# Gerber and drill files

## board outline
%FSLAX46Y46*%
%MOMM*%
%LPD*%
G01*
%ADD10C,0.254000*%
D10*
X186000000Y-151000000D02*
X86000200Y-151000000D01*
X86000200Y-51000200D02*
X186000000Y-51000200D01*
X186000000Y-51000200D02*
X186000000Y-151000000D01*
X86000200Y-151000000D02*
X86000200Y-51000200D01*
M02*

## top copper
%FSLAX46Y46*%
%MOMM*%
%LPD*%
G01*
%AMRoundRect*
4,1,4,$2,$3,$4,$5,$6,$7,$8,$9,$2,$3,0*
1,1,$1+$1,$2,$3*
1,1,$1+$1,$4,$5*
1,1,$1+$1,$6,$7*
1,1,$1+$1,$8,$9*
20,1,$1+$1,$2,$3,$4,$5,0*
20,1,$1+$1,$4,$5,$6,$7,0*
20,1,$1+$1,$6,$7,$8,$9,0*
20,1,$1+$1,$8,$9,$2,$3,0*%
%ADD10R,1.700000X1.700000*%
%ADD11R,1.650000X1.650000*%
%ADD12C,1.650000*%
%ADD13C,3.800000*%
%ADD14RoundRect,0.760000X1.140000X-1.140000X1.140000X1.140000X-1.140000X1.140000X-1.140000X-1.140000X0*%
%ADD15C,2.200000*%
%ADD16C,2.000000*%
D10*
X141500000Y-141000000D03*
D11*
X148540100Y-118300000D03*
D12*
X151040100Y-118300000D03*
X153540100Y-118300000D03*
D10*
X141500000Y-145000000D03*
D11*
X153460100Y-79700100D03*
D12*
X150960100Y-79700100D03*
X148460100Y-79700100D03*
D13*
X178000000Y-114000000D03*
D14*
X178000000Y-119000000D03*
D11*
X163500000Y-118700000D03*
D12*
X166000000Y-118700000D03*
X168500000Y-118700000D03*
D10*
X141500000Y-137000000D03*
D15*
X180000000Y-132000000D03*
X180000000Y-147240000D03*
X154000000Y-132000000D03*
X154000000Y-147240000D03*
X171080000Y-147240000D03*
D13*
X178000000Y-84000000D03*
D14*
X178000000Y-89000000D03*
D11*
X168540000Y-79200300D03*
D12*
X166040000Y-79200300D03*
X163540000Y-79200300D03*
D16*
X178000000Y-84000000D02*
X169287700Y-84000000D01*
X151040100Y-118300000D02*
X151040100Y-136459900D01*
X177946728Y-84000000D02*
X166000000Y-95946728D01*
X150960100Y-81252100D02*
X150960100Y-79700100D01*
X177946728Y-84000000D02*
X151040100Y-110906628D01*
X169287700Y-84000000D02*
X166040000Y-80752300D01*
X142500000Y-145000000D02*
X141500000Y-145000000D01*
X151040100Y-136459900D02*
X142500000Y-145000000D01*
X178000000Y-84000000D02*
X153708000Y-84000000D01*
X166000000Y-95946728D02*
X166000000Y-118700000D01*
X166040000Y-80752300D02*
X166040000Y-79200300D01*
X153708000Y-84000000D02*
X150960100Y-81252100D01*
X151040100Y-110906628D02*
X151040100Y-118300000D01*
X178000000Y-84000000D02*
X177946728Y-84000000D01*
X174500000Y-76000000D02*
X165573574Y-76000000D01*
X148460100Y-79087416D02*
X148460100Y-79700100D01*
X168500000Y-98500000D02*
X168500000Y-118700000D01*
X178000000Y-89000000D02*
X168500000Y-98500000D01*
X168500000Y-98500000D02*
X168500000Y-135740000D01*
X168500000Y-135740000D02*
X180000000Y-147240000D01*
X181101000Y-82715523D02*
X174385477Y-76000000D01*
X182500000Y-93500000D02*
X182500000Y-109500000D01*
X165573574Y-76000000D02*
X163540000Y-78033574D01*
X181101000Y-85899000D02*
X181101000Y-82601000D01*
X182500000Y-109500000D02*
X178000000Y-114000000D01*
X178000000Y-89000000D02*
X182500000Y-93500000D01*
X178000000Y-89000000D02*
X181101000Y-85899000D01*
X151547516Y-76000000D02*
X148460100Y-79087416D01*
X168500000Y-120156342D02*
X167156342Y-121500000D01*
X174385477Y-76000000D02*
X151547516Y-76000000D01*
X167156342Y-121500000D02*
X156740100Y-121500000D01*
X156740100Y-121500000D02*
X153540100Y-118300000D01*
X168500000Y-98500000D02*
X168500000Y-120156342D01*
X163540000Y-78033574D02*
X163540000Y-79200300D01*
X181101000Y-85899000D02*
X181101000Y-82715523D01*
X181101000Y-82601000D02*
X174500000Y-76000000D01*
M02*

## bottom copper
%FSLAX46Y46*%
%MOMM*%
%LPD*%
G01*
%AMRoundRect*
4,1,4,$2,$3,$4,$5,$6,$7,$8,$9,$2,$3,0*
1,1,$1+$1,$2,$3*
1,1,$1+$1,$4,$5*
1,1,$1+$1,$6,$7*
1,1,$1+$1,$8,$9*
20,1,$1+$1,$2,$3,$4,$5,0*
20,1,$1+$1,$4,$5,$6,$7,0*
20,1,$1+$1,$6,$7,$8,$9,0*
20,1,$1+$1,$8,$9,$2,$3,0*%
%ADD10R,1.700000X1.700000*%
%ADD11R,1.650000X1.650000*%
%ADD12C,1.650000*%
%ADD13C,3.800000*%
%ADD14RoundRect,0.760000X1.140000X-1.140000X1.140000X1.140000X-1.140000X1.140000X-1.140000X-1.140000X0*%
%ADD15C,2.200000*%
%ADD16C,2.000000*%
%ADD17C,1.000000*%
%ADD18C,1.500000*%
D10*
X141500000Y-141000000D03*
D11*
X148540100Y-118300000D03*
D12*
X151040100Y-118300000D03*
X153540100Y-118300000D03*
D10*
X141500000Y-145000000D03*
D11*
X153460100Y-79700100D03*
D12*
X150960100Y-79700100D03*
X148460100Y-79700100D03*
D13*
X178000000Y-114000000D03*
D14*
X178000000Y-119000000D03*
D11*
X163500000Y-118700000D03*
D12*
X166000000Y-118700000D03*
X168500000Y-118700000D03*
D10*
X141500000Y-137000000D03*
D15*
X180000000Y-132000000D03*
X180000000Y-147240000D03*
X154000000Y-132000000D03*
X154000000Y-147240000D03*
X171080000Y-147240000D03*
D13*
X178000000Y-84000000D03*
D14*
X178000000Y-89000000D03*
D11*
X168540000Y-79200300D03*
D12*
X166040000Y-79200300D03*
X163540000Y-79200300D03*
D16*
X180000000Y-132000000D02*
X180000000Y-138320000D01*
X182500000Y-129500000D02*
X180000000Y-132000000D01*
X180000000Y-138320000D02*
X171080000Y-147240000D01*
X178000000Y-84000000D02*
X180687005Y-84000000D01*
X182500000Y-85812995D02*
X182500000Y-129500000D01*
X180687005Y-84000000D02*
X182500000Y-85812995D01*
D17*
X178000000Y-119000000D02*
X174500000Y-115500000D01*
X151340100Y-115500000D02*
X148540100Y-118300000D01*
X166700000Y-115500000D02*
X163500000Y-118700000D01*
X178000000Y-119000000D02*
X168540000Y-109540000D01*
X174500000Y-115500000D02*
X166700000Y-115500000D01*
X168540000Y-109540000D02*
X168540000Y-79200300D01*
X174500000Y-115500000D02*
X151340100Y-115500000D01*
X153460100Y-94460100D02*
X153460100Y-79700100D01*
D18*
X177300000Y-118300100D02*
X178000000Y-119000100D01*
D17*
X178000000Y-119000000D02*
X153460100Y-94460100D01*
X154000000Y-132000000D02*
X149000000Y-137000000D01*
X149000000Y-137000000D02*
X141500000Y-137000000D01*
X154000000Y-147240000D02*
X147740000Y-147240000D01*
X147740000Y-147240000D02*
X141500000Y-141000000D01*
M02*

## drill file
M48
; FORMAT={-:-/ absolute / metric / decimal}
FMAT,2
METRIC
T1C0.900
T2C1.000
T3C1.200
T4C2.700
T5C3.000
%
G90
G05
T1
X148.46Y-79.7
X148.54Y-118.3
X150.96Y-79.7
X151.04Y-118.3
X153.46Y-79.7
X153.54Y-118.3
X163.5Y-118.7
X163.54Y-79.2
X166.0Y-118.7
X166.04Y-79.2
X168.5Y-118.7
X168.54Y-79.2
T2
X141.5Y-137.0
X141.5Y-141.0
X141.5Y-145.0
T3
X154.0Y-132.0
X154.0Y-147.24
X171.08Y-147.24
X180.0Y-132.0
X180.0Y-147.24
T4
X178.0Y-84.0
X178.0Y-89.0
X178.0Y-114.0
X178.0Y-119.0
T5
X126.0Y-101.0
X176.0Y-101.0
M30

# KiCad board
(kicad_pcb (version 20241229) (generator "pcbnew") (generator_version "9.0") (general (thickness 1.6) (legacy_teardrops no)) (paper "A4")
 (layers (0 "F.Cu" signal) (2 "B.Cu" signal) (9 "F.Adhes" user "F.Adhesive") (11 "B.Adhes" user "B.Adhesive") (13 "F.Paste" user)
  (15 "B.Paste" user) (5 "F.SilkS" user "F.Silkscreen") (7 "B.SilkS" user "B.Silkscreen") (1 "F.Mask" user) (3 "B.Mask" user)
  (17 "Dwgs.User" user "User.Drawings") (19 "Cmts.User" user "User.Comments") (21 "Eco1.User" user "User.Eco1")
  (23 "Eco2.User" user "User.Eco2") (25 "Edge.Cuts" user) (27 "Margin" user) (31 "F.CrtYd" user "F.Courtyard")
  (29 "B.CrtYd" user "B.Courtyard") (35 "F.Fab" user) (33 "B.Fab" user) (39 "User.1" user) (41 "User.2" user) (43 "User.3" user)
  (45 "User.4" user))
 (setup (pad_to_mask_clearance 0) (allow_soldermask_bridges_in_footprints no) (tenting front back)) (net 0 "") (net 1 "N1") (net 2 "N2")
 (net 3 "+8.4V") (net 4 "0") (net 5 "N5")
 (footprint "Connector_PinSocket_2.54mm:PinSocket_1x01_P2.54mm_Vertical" (layer "F.Cu") (at 141.5 141 90)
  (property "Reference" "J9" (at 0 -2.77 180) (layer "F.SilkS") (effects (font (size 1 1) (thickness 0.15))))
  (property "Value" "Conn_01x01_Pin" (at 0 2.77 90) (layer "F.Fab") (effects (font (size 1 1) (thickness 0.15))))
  (pad "1" thru_hole rect (at 0 0 90) (size 1.7 1.7) (drill 1) (layers "*.Cu" "*.Mask") (remove_unused_layers no) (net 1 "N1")))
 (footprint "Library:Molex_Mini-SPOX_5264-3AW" (layer "F.Cu") (at 148.5401 118.3)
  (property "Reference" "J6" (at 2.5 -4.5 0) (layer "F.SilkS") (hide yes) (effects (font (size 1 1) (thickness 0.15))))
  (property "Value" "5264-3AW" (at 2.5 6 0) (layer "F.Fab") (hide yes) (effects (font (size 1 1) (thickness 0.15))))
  (pad "1" thru_hole rect (at 0 0) (size 1.65 1.65) (drill 0.9) (layers "*.Cu" "*.Mask") (remove_unused_layers no) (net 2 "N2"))
  (pad "2" thru_hole circle (at 2.5 0) (size 1.65 1.65) (drill 0.9) (layers "*.Cu" "*.Mask") (remove_unused_layers no) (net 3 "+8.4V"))
  (pad "3" thru_hole circle (at 5 0) (size 1.65 1.65) (drill 0.9) (layers "*.Cu" "*.Mask") (remove_unused_layers no) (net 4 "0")))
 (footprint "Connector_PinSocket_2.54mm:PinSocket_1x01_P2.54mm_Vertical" (layer "F.Cu") (at 141.5 145 90)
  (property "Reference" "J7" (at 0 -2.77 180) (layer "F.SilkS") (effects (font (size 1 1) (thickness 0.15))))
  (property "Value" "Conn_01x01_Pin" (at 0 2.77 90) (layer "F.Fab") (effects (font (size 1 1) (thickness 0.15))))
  (pad "1" thru_hole rect (at 0 0 90) (size 1.7 1.7) (drill 1) (layers "*.Cu" "*.Mask") (remove_unused_layers no) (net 3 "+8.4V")))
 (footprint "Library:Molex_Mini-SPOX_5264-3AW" (layer "F.Cu") (at 153.4601 79.7001 180)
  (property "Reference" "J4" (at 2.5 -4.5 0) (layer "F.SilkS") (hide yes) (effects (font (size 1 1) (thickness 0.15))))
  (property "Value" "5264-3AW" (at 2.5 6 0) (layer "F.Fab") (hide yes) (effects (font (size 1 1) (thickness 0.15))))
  (pad "1" thru_hole rect (at 0 0 180) (size 1.65 1.65) (drill 0.9) (layers "*.Cu" "*.Mask") (remove_unused_layers no) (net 2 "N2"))
  (pad "2" thru_hole circle (at 2.5 0 180) (size 1.65 1.65) (drill 0.9) (layers "*.Cu" "*.Mask") (remove_unused_layers no) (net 3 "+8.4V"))
  (pad "3" thru_hole circle (at 5 0 180) (size 1.65 1.65) (drill 0.9) (layers "*.Cu" "*.Mask") (remove_unused_layers no) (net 4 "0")))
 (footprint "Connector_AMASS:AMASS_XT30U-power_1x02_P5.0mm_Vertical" (layer "F.Cu") (at 178 119 90)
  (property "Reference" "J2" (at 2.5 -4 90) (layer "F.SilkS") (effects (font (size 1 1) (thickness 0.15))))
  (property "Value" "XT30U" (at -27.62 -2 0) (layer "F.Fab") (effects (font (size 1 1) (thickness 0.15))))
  (pad "1" thru_hole circle (at 5 0 90) (size 3.8 3.8) (drill 2.7) (layers "*.Cu" "*.Mask") (remove_unused_layers no) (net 4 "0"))
  (pad "2" thru_hole roundrect (at 0 0 90) (size 3.8 3.8) (drill 2.7) (layers "*.Cu" "*.Mask") (remove_unused_layers no)
   (roundrect_rratio 0.2) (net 2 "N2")))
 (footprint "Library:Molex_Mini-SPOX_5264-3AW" (layer "F.Cu") (at 163.5 118.7)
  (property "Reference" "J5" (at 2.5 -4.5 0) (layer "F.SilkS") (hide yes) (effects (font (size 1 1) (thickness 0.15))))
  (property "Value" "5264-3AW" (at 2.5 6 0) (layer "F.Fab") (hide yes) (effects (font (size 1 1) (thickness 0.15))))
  (pad "1" thru_hole rect (at 0 0) (size 1.65 1.65) (drill 0.9) (layers "*.Cu" "*.Mask") (remove_unused_layers no) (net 2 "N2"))
  (pad "2" thru_hole circle (at 2.5 0) (size 1.65 1.65) (drill 0.9) (layers "*.Cu" "*.Mask") (remove_unused_layers no) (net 3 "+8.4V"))
  (pad "3" thru_hole circle (at 5 0) (size 1.65 1.65) (drill 0.9) (layers "*.Cu" "*.Mask") (remove_unused_layers no) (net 4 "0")))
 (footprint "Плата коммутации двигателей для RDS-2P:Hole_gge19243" (layer "F.Cu") (at 126.0001 101.0001)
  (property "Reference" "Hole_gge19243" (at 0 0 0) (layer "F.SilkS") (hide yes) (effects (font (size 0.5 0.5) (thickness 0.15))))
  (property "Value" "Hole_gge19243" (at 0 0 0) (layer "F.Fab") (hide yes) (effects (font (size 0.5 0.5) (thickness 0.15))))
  (pad "" np_thru_hole circle (at 0 0) (size 3 3) (drill 3) (layers "*.Cu" "*.Mask")))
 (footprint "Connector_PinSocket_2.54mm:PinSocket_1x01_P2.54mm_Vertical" (layer "F.Cu") (at 141.5 137 90)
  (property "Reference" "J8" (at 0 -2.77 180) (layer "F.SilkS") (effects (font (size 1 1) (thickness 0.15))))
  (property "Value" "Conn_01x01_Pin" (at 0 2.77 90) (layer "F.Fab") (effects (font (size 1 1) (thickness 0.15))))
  (pad "1" thru_hole rect (at 0 0 90) (size 1.7 1.7) (drill 1) (layers "*.Cu" "*.Mask") (remove_unused_layers no) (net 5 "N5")))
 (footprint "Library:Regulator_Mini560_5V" (layer "F.Cu") (at 180 132 180)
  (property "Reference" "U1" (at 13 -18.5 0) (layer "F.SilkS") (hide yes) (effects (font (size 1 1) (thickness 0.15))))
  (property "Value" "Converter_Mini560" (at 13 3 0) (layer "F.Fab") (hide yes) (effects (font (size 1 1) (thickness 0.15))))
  (pad "1" thru_hole circle (at 0 0 180) (size 2.2 2.2) (drill 1.2) (layers "*.Cu" "*.Mask") (remove_unused_layers no) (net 3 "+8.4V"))
  (pad "2" thru_hole circle (at 0 -15.24 180) (size 2.2 2.2) (drill 1.2) (layers "*.Cu" "*.Mask") (remove_unused_layers no) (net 4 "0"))
  (pad "3" thru_hole circle (at 26 0 180) (size 2.2 2.2) (drill 1.2) (layers "*.Cu" "*.Mask") (remove_unused_layers no) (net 5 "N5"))
  (pad "4" thru_hole circle (at 26 -15.24 180) (size 2.2 2.2) (drill 1.2) (layers "*.Cu" "*.Mask") (remove_unused_layers no) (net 1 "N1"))
  (pad "5" thru_hole circle (at 8.92 -15.24 180) (size 2.2 2.2) (drill 1.2) (layers "*.Cu" "*.Mask") (remove_unused_layers no)
   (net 3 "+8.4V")))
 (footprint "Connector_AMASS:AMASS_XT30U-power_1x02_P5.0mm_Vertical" (layer "F.Cu") (at 178 89 90)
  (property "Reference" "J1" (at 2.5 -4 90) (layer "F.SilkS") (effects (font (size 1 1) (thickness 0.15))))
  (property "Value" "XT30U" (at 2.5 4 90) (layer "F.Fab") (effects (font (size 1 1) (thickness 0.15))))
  (pad "1" thru_hole circle (at 5 0 90) (size 3.8 3.8) (drill 2.7) (layers "*.Cu" "*.Mask") (remove_unused_layers no) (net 3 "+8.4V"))
  (pad "2" thru_hole roundrect (at 0 0 90) (size 3.8 3.8) (drill 2.7) (layers "*.Cu" "*.Mask") (remove_unused_layers no)
   (roundrect_rratio 0.2) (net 4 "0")))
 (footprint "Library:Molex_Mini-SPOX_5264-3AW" (layer "F.Cu") (at 168.54 79.2003 180)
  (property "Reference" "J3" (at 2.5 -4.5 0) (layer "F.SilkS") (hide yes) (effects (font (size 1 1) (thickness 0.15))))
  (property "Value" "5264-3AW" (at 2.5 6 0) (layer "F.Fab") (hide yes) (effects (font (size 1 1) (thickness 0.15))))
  (pad "1" thru_hole rect (at 0 0 180) (size 1.65 1.65) (drill 0.9) (layers "*.Cu" "*.Mask") (remove_unused_layers no) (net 2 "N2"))
  (pad "2" thru_hole circle (at 2.5 0 180) (size 1.65 1.65) (drill 0.9) (layers "*.Cu" "*.Mask") (remove_unused_layers no) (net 3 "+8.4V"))
  (pad "3" thru_hole circle (at 5 0 180) (size 1.65 1.65) (drill 0.9) (layers "*.Cu" "*.Mask") (remove_unused_layers no) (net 4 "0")))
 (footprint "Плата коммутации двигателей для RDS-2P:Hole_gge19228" (layer "F.Cu") (at 176 101.0001)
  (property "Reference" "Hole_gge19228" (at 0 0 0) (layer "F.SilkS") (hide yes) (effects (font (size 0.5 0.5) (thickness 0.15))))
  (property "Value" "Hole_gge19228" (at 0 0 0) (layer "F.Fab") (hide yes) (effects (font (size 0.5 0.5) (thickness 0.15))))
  (pad "" np_thru_hole circle (at 0 0) (size 3 3) (drill 3) (layers "*.Cu" "*.Mask")))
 (gr_line (start 186 151) (end 86.0002 151) (stroke (width 0.254) (type default)) (layer "Edge.Cuts"))
 (gr_line (start 86.0002 51.0002) (end 186 51.0002) (stroke (width 0.254) (type default)) (layer "Edge.Cuts"))
 (gr_line (start 186 51.0002) (end 186 151) (stroke (width 0.254) (type default)) (layer "Edge.Cuts"))
 (gr_line (start 86.0002 151) (end 86.0002 51.0002) (stroke (width 0.254) (type default)) (layer "Edge.Cuts"))
 (segment (start 178 84) (end 169.2877 84) (width 2) (layer "F.Cu") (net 3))
 (segment (start 151.0401 118.3) (end 151.0401 136.4599) (width 2) (layer "F.Cu") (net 3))
 (segment (start 177.946728 84) (end 166 95.946728) (width 2) (layer "F.Cu") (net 3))
 (segment (start 150.9601 81.2521) (end 150.9601 79.7001) (width 2) (layer "F.Cu") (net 3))
 (segment (start 177.946728 84) (end 151.0401 110.906628) (width 2) (layer "F.Cu") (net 3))
 (segment (start 169.2877 84) (end 166.04 80.7523) (width 2) (layer "F.Cu") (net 3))
 (segment (start 142.5 145) (end 141.5 145) (width 2) (layer "F.Cu") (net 3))
 (segment (start 151.0401 136.4599) (end 142.5 145) (width 2) (layer "F.Cu") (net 3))
 (segment (start 178 84) (end 153.708 84) (width 2) (layer "F.Cu") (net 3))
 (segment (start 166 95.946728) (end 166 118.7) (width 2) (layer "F.Cu") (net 3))
 (segment (start 166.04 80.7523) (end 166.04 79.2003) (width 2) (layer "F.Cu") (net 3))
 (segment (start 153.708 84) (end 150.9601 81.2521) (width 2) (layer "F.Cu") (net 3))
 (segment (start 151.0401 110.906628) (end 151.0401 118.3) (width 2) (layer "F.Cu") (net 3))
 (segment (start 178 84) (end 177.946728 84) (width 2) (layer "F.Cu") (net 3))
 (segment (start 180 132) (end 180 138.32) (width 2) (layer "B.Cu") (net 3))
 (segment (start 182.5 129.5) (end 180 132) (width 2) (layer "B.Cu") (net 3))
 (segment (start 180 138.32) (end 171.08 147.24) (width 2) (layer "B.Cu") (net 3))
 (segment (start 178 84) (end 180.687005 84) (width 2) (layer "B.Cu") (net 3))
 (segment (start 182.5 85.812995) (end 182.5 129.5) (width 2) (layer "B.Cu") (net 3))
 (segment (start 180.687005 84) (end 182.5 85.812995) (width 2) (layer "B.Cu") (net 3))
 (segment (start 174.5 76) (end 165.573574 76) (width 2) (layer "F.Cu") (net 4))
 (segment (start 148.4601 79.087416) (end 148.4601 79.7001) (width 2) (layer "F.Cu") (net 4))
 (segment (start 168.5 98.5) (end 168.5 118.7) (width 2) (layer "F.Cu") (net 4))
 (segment (start 178 89) (end 168.5 98.5) (width 2) (layer "F.Cu") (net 4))
 (segment (start 168.5 98.5) (end 168.5 135.74) (width 2) (layer "F.Cu") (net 4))
 (segment (start 168.5 135.74) (end 180 147.24) (width 2) (layer "F.Cu") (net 4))
 (segment (start 181.101 82.715523) (end 174.385477 76) (width 2) (layer "F.Cu") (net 4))
 (segment (start 182.5 93.5) (end 182.5 109.5) (width 2) (layer "F.Cu") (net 4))
 (segment (start 165.573574 76) (end 163.54 78.033574) (width 2) (layer "F.Cu") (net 4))
 (segment (start 181.101 85.899) (end 181.101 82.601) (width 2) (layer "F.Cu") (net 4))
 (segment (start 182.5 109.5) (end 178 114) (width 2) (layer "F.Cu") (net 4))
 (segment (start 178 89) (end 182.5 93.5) (width 2) (layer "F.Cu") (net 4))
 (segment (start 178 89) (end 181.101 85.899) (width 2) (layer "F.Cu") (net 4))
 (segment (start 151.547516 76) (end 148.4601 79.087416) (width 2) (layer "F.Cu") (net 4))
 (segment (start 168.5 120.156342) (end 167.156342 121.5) (width 2) (layer "F.Cu") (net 4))
 (segment (start 174.385477 76) (end 151.547516 76) (width 2) (layer "F.Cu") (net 4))
 (segment (start 167.156342 121.5) (end 156.7401 121.5) (width 2) (layer "F.Cu") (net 4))
 (segment (start 156.7401 121.5) (end 153.5401 118.3) (width 2) (layer "F.Cu") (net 4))
 (segment (start 168.5 98.5) (end 168.5 120.156342) (width 2) (layer "F.Cu") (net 4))
 (segment (start 163.54 78.033574) (end 163.54 79.2003) (width 2) (layer "F.Cu") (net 4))
 (segment (start 181.101 85.899) (end 181.101 82.715523) (width 2) (layer "F.Cu") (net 4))
 (segment (start 181.101 82.601) (end 174.5 76) (width 2) (layer "F.Cu") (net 4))
 (segment (start 178 119) (end 174.5 115.5) (width 1) (layer "B.Cu") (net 2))
 (segment (start 151.3401 115.5) (end 148.5401 118.3) (width 1) (layer "B.Cu") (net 2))
 (segment (start 166.7 115.5) (end 163.5 118.7) (width 1) (layer "B.Cu") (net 2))
 (segment (start 178 119) (end 168.54 109.54) (width 1) (layer "B.Cu") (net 2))
 (segment (start 174.5 115.5) (end 166.7 115.5) (width 1) (layer "B.Cu") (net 2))
 (segment (start 168.54 109.54) (end 168.54 79.2003) (width 1) (layer "B.Cu") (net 2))
 (segment (start 174.5 115.5) (end 151.3401 115.5) (width 1) (layer "B.Cu") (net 2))
 (segment (start 153.4601 94.4601) (end 153.4601 79.7001) (width 1) (layer "B.Cu") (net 2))
 (segment (start 177.3 118.3001) (end 178 119.0001) (width 1.5) (layer "B.Cu") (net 2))
 (segment (start 178 119) (end 153.4601 94.4601) (width 1) (layer "B.Cu") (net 2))
 (segment (start 154 132) (end 149 137) (width 1) (layer "B.Cu") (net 5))
 (segment (start 149 137) (end 141.5 137) (width 1) (layer "B.Cu") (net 5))
 (segment (start 154 147.24) (end 147.74 147.24) (width 1) (layer "B.Cu") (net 1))
 (segment (start 147.74 147.24) (end 141.5 141) (width 1) (layer "B.Cu") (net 1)))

